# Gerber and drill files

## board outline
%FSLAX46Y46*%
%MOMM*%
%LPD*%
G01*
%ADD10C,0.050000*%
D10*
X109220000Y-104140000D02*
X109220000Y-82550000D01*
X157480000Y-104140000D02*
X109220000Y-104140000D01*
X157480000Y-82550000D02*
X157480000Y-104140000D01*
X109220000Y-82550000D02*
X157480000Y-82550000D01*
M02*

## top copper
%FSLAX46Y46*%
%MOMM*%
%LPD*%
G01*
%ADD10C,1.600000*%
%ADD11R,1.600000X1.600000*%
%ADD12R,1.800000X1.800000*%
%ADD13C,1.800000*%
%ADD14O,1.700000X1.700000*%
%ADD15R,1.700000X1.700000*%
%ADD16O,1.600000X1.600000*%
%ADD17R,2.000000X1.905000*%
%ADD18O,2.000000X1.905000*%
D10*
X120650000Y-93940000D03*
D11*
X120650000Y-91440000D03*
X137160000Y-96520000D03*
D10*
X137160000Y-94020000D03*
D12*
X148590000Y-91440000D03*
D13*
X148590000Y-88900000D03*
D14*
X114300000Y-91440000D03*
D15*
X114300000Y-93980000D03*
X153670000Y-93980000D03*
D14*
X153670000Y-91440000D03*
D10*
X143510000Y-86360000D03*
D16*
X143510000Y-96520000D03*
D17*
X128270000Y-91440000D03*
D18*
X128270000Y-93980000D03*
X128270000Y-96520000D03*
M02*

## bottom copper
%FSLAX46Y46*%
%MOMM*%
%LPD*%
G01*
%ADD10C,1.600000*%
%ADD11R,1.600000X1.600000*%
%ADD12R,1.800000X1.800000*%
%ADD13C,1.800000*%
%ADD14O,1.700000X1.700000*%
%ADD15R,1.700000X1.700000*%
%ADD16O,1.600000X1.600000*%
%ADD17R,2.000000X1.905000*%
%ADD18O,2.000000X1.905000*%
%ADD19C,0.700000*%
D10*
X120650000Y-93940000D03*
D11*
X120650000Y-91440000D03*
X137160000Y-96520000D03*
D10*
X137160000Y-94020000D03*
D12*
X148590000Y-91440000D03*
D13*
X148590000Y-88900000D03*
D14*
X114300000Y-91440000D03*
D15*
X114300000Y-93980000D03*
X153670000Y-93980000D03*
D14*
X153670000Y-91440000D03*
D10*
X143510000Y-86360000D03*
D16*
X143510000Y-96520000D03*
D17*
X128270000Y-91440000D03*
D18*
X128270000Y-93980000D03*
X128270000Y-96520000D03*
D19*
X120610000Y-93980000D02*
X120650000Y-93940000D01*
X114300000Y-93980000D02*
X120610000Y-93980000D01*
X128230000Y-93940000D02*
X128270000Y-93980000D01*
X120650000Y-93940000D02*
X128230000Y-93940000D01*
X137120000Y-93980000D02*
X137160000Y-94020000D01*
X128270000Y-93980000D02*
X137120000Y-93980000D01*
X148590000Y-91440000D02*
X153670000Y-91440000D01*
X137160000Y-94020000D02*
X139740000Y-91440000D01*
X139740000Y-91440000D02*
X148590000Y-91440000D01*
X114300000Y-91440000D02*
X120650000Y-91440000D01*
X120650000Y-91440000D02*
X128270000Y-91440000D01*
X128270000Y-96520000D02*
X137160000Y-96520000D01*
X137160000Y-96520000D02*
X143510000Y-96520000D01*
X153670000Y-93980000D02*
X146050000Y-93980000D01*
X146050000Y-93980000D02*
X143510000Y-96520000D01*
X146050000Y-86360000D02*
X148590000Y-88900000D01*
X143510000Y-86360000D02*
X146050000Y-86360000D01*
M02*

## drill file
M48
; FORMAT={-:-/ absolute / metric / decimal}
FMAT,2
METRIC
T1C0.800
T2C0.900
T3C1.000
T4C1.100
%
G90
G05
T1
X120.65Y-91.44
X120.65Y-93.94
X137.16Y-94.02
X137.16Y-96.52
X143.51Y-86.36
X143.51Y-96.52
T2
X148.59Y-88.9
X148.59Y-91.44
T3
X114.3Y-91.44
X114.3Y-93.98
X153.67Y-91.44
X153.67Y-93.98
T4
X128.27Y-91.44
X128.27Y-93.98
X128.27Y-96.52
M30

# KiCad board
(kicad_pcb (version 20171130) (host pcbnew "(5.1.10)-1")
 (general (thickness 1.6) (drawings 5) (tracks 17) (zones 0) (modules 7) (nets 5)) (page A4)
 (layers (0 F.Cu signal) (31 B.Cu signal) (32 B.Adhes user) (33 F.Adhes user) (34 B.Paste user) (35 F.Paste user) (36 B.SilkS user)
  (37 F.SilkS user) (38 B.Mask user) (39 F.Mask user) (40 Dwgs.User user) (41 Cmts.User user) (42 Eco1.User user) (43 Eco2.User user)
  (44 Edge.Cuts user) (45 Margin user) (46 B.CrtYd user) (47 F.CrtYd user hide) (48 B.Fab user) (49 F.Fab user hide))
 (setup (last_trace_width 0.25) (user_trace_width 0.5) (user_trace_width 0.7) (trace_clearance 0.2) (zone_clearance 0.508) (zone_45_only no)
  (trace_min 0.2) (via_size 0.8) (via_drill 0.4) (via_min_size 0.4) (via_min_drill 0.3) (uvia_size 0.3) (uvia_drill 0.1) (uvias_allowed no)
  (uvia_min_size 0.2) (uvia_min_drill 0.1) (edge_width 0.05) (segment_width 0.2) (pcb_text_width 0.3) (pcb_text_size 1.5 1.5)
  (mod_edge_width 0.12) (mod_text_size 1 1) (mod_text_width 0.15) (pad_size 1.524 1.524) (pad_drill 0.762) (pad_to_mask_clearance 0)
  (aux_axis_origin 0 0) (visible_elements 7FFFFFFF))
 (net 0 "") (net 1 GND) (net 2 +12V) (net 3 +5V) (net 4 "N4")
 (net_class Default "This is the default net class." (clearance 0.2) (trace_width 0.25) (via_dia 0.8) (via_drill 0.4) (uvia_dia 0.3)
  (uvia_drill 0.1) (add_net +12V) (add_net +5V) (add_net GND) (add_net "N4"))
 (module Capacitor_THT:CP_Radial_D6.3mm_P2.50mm (layer F.Cu) (at 120.65 91.44 270)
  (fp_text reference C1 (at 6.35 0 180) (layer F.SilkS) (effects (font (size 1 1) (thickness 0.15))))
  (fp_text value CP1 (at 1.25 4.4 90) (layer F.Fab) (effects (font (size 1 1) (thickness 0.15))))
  (pad 2 thru_hole circle (at 2.5 0 270) (size 1.6 1.6) (drill 0.8) (layers *.Cu *.Mask) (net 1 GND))
  (pad 1 thru_hole rect (at 0 0 270) (size 1.6 1.6) (drill 0.8) (layers *.Cu *.Mask) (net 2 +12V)))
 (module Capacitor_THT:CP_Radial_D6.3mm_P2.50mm (layer F.Cu) (at 137.16 96.52 90)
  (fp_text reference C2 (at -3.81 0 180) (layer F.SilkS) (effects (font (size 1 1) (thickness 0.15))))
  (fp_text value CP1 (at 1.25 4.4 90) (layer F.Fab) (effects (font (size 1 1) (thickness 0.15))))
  (pad 1 thru_hole rect (at 0 0 90) (size 1.6 1.6) (drill 0.8) (layers *.Cu *.Mask) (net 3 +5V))
  (pad 2 thru_hole circle (at 2.5 0 90) (size 1.6 1.6) (drill 0.8) (layers *.Cu *.Mask) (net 1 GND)))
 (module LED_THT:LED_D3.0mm (layer F.Cu) (at 148.59 91.44 90)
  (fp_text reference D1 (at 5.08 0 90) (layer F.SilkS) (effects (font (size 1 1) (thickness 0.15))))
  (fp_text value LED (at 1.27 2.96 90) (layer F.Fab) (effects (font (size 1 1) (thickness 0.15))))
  (pad 1 thru_hole rect (at 0 0 90) (size 1.8 1.8) (drill 0.9) (layers *.Cu *.Mask) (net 1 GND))
  (pad 2 thru_hole circle (at 2.54 0 90) (size 1.8 1.8) (drill 0.9) (layers *.Cu *.Mask) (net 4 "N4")))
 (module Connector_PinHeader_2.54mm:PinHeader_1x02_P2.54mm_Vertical (layer F.Cu) (at 114.3 93.98 180)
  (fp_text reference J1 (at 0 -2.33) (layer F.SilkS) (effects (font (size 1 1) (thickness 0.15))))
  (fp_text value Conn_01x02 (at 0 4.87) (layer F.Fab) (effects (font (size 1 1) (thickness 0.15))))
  (pad 2 thru_hole oval (at 0 2.54 180) (size 1.7 1.7) (drill 1) (layers *.Cu *.Mask) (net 2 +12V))
  (pad 1 thru_hole rect (at 0 0 180) (size 1.7 1.7) (drill 1) (layers *.Cu *.Mask) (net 1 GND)))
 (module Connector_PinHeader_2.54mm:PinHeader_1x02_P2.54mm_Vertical (layer F.Cu) (at 153.67 93.98 180)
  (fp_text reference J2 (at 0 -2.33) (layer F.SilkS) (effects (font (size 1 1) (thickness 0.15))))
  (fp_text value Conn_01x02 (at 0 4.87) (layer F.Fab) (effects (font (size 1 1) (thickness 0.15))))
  (pad 1 thru_hole rect (at 0 0 180) (size 1.7 1.7) (drill 1) (layers *.Cu *.Mask) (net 3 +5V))
  (pad 2 thru_hole oval (at 0 2.54 180) (size 1.7 1.7) (drill 1) (layers *.Cu *.Mask) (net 1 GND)))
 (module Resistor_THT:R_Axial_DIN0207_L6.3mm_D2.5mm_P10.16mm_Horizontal (layer F.Cu) (at 143.51 86.36 270)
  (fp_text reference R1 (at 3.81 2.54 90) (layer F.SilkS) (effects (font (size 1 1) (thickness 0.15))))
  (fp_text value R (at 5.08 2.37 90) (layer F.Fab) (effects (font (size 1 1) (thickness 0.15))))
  (pad 1 thru_hole circle (at 0 0 270) (size 1.6 1.6) (drill 0.8) (layers *.Cu *.Mask) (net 4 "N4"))
  (pad 2 thru_hole oval (at 10.16 0 270) (size 1.6 1.6) (drill 0.8) (layers *.Cu *.Mask) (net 3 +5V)))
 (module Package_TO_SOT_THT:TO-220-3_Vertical (layer F.Cu) (at 128.27 91.44 270)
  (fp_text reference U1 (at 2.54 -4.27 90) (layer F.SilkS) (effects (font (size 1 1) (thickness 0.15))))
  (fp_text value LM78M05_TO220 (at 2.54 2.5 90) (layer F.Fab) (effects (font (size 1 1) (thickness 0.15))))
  (pad 1 thru_hole rect (at 0 0 270) (size 1.905 2) (drill 1.1) (layers *.Cu *.Mask) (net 2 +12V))
  (pad 2 thru_hole oval (at 2.54 0 270) (size 1.905 2) (drill 1.1) (layers *.Cu *.Mask) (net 1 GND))
  (pad 3 thru_hole oval (at 5.08 0 270) (size 1.905 2) (drill 1.1) (layers *.Cu *.Mask) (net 3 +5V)))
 (gr_line (start 109.22 104.14) (end 109.22 82.55) (layer Edge.Cuts) (width 0.05))
 (gr_line (start 157.48 104.14) (end 109.22 104.14) (layer Edge.Cuts) (width 0.05))
 (gr_line (start 157.48 82.55) (end 157.48 104.14) (layer Edge.Cuts) (width 0.05))
 (gr_line (start 109.22 82.55) (end 157.48 82.55) (layer Edge.Cuts) (width 0.05))
 (segment (start 120.61 93.98) (end 120.65 93.94) (width 0.7) (layer B.Cu) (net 1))
 (segment (start 114.3 93.98) (end 120.61 93.98) (width 0.7) (layer B.Cu) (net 1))
 (segment (start 128.23 93.94) (end 128.27 93.98) (width 0.7) (layer B.Cu) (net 1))
 (segment (start 120.65 93.94) (end 128.23 93.94) (width 0.7) (layer B.Cu) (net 1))
 (segment (start 137.12 93.98) (end 137.16 94.02) (width 0.7) (layer B.Cu) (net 1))
 (segment (start 128.27 93.98) (end 137.12 93.98) (width 0.7) (layer B.Cu) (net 1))
 (segment (start 148.59 91.44) (end 153.67 91.44) (width 0.7) (layer B.Cu) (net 1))
 (segment (start 137.16 94.02) (end 139.74 91.44) (width 0.7) (layer B.Cu) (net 1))
 (segment (start 139.74 91.44) (end 148.59 91.44) (width 0.7) (layer B.Cu) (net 1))
 (segment (start 114.3 91.44) (end 120.65 91.44) (width 0.7) (layer B.Cu) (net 2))
 (segment (start 120.65 91.44) (end 128.27 91.44) (width 0.7) (layer B.Cu) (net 2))
 (segment (start 128.27 96.52) (end 137.16 96.52) (width 0.7) (layer B.Cu) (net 3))
 (segment (start 137.16 96.52) (end 143.51 96.52) (width 0.7) (layer B.Cu) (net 3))
 (segment (start 153.67 93.98) (end 146.05 93.98) (width 0.7) (layer B.Cu) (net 3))
 (segment (start 146.05 93.98) (end 143.51 96.52) (width 0.7) (layer B.Cu) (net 3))
 (segment (start 146.05 86.36) (end 148.59 88.9) (width 0.7) (layer B.Cu) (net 4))
 (segment (start 143.51 86.36) (end 146.05 86.36) (width 0.7) (layer B.Cu) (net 4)))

